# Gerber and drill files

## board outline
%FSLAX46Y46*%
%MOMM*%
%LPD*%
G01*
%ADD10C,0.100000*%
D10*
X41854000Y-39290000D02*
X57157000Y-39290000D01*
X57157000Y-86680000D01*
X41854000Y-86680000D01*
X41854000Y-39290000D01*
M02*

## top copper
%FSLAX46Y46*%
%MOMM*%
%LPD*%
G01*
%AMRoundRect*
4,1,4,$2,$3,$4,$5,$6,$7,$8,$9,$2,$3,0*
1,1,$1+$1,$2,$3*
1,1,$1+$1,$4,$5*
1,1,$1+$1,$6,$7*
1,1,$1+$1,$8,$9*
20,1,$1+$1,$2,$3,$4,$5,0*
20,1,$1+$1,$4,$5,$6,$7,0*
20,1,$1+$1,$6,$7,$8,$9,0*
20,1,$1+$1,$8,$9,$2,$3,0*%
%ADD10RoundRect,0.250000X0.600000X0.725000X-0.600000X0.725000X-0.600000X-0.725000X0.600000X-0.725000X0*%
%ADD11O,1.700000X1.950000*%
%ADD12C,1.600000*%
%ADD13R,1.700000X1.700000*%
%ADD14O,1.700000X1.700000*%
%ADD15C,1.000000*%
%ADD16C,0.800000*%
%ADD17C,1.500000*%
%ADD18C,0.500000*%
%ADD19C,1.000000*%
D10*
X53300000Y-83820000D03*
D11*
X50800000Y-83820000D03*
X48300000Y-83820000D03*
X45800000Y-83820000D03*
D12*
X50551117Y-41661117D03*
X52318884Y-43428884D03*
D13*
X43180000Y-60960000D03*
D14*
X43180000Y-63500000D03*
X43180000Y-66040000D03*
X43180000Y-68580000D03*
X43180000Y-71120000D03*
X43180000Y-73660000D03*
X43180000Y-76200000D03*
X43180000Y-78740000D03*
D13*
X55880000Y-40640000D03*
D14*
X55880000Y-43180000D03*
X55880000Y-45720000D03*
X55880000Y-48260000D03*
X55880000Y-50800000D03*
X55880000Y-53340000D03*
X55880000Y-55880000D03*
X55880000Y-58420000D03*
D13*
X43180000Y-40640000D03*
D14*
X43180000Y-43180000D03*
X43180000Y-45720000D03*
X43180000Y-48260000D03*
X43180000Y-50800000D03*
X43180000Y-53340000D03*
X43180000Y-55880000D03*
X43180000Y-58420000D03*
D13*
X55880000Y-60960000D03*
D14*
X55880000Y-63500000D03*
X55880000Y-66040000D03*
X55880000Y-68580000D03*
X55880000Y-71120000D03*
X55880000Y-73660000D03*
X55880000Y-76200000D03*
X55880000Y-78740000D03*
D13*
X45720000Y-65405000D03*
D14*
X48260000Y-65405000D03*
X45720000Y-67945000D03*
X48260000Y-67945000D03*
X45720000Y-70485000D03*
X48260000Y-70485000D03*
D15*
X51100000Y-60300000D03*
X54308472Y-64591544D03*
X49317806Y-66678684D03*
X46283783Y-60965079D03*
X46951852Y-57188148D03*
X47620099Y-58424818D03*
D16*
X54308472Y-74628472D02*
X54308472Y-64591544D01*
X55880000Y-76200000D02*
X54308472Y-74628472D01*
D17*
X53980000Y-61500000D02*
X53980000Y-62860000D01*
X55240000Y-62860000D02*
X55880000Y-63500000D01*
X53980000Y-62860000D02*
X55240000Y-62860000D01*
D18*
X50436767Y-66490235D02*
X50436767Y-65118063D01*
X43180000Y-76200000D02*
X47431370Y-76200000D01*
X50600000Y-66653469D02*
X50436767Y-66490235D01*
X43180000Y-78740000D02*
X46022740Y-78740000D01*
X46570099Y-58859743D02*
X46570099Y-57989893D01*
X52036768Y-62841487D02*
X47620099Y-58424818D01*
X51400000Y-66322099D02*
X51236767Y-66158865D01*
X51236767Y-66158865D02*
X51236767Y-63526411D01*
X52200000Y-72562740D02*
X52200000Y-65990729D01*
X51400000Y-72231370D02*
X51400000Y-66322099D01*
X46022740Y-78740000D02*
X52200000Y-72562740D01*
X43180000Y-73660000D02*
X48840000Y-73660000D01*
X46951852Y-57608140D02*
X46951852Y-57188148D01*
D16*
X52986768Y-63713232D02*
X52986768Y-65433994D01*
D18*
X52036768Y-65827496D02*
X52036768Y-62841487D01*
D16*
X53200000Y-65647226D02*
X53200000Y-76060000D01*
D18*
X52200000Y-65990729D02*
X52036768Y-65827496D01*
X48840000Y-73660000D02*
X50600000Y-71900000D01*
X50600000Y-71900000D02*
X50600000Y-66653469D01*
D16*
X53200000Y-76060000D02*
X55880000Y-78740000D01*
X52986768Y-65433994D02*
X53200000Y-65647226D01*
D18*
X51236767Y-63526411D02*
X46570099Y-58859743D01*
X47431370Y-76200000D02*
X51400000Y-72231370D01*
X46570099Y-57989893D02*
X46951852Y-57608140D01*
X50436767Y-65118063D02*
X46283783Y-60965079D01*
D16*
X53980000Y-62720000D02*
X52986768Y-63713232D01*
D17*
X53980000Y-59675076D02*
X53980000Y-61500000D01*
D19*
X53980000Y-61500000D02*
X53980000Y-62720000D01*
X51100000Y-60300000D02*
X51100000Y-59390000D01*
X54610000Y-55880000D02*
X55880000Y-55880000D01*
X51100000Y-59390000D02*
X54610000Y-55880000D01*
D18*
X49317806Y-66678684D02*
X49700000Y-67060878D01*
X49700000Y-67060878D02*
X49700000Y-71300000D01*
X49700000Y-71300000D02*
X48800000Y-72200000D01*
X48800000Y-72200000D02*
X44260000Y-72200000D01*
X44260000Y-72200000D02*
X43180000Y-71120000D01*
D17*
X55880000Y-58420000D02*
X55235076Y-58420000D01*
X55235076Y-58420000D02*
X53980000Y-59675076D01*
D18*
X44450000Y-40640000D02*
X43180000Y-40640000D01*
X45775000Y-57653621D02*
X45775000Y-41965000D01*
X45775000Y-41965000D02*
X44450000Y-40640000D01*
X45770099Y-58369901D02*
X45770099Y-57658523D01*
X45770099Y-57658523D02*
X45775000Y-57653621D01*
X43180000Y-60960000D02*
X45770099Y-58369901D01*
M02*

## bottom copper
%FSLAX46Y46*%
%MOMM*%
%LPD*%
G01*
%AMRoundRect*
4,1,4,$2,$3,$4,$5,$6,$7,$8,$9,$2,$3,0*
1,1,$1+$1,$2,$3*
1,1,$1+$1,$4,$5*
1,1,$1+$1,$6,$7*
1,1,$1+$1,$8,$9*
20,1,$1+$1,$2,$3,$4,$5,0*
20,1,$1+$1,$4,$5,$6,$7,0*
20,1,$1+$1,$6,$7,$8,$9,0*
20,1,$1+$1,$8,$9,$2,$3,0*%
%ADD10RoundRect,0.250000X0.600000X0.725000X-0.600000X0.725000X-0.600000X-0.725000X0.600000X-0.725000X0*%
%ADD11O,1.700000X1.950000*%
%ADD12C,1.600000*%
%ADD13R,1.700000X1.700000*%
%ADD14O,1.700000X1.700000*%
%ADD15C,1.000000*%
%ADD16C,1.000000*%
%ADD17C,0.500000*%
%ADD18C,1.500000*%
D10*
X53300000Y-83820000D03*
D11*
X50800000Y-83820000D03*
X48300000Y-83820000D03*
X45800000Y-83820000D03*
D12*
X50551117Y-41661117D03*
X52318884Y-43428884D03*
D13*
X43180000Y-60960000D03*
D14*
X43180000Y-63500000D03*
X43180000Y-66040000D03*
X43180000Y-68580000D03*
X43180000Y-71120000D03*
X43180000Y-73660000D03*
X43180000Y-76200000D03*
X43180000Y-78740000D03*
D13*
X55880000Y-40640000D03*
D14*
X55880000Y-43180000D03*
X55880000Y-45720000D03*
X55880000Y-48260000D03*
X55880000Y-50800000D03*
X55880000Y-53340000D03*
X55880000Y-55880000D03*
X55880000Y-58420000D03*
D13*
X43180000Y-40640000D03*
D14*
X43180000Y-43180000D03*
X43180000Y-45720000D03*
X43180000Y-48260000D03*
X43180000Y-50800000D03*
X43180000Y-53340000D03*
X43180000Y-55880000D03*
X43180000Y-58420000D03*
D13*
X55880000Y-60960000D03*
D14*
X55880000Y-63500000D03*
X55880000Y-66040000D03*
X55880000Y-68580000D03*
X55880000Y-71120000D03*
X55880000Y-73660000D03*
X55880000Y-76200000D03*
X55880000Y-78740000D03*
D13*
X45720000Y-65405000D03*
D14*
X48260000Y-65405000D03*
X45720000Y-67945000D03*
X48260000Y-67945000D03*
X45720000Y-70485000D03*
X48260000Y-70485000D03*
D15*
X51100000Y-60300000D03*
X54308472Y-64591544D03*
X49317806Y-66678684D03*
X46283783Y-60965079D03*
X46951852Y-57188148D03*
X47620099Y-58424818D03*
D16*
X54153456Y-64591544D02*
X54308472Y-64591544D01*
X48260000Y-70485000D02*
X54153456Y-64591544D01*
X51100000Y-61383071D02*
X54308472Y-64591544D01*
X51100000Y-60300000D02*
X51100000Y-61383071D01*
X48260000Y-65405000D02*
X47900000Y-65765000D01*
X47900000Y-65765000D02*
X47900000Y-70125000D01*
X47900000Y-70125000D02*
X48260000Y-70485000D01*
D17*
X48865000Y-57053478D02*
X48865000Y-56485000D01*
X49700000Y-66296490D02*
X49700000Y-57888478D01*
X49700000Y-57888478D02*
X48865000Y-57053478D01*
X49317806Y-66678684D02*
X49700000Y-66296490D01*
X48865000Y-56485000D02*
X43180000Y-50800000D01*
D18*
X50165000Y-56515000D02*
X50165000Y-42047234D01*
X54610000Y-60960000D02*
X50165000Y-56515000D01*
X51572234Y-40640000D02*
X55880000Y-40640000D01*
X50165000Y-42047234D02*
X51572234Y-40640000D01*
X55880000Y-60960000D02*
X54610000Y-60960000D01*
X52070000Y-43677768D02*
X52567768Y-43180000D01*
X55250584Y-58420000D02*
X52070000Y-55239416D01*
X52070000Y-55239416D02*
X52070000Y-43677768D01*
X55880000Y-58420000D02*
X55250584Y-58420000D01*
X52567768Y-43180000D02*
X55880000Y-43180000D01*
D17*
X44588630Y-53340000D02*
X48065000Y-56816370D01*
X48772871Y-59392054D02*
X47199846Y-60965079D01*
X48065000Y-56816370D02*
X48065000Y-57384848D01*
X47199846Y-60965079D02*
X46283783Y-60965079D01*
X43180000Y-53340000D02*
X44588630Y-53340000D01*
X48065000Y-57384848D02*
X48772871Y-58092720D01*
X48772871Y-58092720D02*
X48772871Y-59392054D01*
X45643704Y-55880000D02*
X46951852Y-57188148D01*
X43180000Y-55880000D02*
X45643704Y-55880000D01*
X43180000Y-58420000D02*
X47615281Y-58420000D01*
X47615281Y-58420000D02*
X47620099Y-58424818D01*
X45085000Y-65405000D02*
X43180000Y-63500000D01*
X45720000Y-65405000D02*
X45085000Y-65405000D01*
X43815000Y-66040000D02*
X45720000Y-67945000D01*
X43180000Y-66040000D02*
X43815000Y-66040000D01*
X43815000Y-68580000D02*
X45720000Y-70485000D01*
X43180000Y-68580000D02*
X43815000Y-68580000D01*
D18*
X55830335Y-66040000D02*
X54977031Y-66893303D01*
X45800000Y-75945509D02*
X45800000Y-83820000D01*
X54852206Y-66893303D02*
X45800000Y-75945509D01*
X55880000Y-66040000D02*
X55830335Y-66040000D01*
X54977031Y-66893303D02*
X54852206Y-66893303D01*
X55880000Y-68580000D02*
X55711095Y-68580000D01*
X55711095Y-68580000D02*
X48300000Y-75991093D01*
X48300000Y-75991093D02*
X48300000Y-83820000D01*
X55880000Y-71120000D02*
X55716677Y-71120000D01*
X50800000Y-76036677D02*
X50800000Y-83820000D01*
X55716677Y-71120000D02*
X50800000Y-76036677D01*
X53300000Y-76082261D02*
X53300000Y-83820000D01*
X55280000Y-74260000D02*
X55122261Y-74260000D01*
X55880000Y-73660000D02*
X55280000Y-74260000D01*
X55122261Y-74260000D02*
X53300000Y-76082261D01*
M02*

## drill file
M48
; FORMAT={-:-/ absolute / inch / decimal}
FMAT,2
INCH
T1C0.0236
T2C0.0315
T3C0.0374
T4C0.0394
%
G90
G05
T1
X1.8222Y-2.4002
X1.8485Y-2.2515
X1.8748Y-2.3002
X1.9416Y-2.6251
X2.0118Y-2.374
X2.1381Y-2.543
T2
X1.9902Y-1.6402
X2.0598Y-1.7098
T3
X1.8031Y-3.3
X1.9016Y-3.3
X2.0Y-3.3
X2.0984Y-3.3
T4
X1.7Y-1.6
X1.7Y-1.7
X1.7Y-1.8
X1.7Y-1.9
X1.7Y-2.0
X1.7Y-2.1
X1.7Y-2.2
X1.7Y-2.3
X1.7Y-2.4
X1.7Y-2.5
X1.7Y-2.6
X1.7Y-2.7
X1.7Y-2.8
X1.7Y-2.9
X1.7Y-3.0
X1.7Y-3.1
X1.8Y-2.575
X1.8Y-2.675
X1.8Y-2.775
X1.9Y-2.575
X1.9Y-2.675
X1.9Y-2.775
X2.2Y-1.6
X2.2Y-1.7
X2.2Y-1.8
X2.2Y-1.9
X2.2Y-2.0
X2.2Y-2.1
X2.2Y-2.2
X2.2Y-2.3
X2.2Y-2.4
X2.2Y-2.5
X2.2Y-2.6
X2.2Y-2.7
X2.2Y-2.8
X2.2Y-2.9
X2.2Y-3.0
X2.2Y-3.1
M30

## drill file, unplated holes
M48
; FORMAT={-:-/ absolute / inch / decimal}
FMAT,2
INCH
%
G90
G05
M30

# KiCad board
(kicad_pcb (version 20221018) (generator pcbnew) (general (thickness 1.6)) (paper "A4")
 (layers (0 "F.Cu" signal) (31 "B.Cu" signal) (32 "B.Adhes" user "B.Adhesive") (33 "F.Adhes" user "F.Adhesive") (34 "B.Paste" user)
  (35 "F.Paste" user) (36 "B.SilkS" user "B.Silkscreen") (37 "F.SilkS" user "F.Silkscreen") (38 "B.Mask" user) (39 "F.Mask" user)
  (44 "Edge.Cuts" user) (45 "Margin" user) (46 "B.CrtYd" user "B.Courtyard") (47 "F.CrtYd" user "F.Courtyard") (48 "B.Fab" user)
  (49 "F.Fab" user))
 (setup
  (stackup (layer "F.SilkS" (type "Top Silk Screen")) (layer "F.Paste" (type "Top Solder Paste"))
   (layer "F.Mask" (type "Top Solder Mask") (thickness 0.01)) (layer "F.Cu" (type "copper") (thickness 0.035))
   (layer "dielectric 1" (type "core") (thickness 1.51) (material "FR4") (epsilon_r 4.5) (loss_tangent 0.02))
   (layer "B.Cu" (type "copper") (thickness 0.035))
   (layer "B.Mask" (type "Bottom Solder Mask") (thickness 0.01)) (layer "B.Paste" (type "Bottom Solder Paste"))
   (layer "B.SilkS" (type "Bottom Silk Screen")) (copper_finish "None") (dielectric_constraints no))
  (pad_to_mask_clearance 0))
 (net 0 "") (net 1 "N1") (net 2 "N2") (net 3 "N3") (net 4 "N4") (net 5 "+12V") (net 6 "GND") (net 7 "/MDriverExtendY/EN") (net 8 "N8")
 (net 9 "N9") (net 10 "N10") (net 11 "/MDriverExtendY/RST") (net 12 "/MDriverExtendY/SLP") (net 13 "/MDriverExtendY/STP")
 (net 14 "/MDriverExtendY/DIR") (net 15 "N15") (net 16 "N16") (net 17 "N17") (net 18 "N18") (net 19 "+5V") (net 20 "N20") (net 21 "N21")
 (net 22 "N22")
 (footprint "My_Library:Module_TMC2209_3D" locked (layer "F.Cu") (at 43.18 40.64)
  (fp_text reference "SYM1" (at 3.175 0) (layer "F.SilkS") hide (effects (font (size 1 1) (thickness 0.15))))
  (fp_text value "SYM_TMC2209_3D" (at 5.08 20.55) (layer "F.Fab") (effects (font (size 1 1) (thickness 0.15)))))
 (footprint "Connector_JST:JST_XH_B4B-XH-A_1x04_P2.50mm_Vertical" (layer "F.Cu") (at 53.3 83.82 180)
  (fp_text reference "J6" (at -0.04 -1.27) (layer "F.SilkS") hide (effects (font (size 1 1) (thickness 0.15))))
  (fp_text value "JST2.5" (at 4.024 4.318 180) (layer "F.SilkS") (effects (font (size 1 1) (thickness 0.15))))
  (pad "1" thru_hole roundrect (at 0 0 180) (size 1.7 1.95) (drill 0.95) (layers "*.Cu" "*.Mask") (roundrect_rratio 0.1470588235)
   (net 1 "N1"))
  (pad "2" thru_hole oval (at 2.5 0 180) (size 1.7 1.95) (drill 0.95) (layers "*.Cu" "*.Mask") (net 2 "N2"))
  (pad "3" thru_hole oval (at 5 0 180) (size 1.7 1.95) (drill 0.95) (layers "*.Cu" "*.Mask") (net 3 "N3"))
  (pad "4" thru_hole oval (at 7.5 0 180) (size 1.7 1.95) (drill 0.95) (layers "*.Cu" "*.Mask") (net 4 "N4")))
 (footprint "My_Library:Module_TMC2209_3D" (layer "F.Cu") (at 43.18 60.96)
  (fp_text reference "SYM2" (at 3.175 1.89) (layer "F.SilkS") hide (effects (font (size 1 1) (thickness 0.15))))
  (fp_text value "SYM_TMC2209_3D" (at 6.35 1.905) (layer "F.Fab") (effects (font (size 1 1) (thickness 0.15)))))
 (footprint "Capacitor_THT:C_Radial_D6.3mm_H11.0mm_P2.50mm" (layer "F.Cu") (at 50.551117 41.661117 -45)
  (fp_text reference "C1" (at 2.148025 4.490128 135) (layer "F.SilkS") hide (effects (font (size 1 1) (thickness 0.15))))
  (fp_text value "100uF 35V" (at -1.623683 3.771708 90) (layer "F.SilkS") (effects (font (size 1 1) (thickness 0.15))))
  (pad "1" thru_hole circle (at 0 0 315) (size 1.6 1.6) (drill 0.8) (layers "*.Cu" "*.Mask") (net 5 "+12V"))
  (pad "2" thru_hole circle (at 2.5 0 315) (size 1.6 1.6) (drill 0.8) (layers "*.Cu" "*.Mask") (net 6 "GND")))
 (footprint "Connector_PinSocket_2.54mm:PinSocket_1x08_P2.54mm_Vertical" (layer "F.Cu") (at 43.18 60.96)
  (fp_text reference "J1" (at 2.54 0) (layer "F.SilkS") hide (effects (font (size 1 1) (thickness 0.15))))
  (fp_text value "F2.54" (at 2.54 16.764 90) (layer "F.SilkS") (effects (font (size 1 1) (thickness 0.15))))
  (pad "1" thru_hole rect (at 0 0) (size 1.7 1.7) (drill 1) (layers "*.Cu" "*.Mask") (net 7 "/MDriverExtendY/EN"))
  (pad "2" thru_hole oval (at 0 2.54) (size 1.7 1.7) (drill 1) (layers "*.Cu" "*.Mask") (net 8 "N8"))
  (pad "3" thru_hole oval (at 0 5.08) (size 1.7 1.7) (drill 1) (layers "*.Cu" "*.Mask") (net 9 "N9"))
  (pad "4" thru_hole oval (at 0 7.62) (size 1.7 1.7) (drill 1) (layers "*.Cu" "*.Mask") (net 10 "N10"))
  (pad "5" thru_hole oval (at 0 10.16) (size 1.7 1.7) (drill 1) (layers "*.Cu" "*.Mask") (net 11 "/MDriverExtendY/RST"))
  (pad "6" thru_hole oval (at 0 12.7) (size 1.7 1.7) (drill 1) (layers "*.Cu" "*.Mask") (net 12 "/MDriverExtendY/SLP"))
  (pad "7" thru_hole oval (at 0 15.24) (size 1.7 1.7) (drill 1) (layers "*.Cu" "*.Mask") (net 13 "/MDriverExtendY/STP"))
  (pad "8" thru_hole oval (at 0 17.78) (size 1.7 1.7) (drill 1) (layers "*.Cu" "*.Mask") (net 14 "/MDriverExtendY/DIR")))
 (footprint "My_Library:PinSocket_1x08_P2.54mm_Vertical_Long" (layer "F.Cu") (at 55.88 40.64)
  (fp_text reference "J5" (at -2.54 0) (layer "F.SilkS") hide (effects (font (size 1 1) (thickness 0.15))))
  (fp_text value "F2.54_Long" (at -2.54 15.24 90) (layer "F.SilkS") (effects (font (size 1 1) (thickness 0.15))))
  (pad "1" thru_hole rect (at 0 0) (size 1.7 1.7) (drill 1) (layers "*.Cu" "*.Mask") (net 5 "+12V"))
  (pad "2" thru_hole oval (at 0 2.54) (size 1.7 1.7) (drill 1) (layers "*.Cu" "*.Mask") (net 6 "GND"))
  (pad "3" thru_hole oval (at 0 5.08) (size 1.7 1.7) (drill 1) (layers "*.Cu" "*.Mask") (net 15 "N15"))
  (pad "4" thru_hole oval (at 0 7.62) (size 1.7 1.7) (drill 1) (layers "*.Cu" "*.Mask") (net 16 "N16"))
  (pad "5" thru_hole oval (at 0 10.16) (size 1.7 1.7) (drill 1) (layers "*.Cu" "*.Mask") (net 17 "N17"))
  (pad "6" thru_hole oval (at 0 12.7) (size 1.7 1.7) (drill 1) (layers "*.Cu" "*.Mask") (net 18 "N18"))
  (pad "7" thru_hole oval (at 0 15.24) (size 1.7 1.7) (drill 1) (layers "*.Cu" "*.Mask") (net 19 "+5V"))
  (pad "8" thru_hole oval (at 0 17.78) (size 1.7 1.7) (drill 1) (layers "*.Cu" "*.Mask") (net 6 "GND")))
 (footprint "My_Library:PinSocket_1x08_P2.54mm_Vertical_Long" (layer "F.Cu") (at 43.18 40.64)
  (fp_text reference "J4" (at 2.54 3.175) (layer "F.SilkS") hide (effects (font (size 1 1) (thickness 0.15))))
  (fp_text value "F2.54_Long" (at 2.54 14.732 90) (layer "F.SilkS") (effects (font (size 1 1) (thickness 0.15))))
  (pad "1" thru_hole rect (at 0 0) (size 1.7 1.7) (drill 1) (layers "*.Cu" "*.Mask") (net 7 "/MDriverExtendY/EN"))
  (pad "2" thru_hole oval (at 0 2.54) (size 1.7 1.7) (drill 1) (layers "*.Cu" "*.Mask") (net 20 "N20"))
  (pad "3" thru_hole oval (at 0 5.08) (size 1.7 1.7) (drill 1) (layers "*.Cu" "*.Mask") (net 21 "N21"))
  (pad "4" thru_hole oval (at 0 7.62) (size 1.7 1.7) (drill 1) (layers "*.Cu" "*.Mask") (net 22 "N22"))
  (pad "5" thru_hole oval (at 0 10.16) (size 1.7 1.7) (drill 1) (layers "*.Cu" "*.Mask") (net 11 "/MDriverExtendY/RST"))
  (pad "6" thru_hole oval (at 0 12.7) (size 1.7 1.7) (drill 1) (layers "*.Cu" "*.Mask") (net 12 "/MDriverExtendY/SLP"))
  (pad "7" thru_hole oval (at 0 15.24) (size 1.7 1.7) (drill 1) (layers "*.Cu" "*.Mask") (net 13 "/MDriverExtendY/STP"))
  (pad "8" thru_hole oval (at 0 17.78) (size 1.7 1.7) (drill 1) (layers "*.Cu" "*.Mask") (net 14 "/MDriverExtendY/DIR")))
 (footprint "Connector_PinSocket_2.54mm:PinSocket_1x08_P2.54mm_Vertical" (layer "F.Cu") (at 55.88 60.96)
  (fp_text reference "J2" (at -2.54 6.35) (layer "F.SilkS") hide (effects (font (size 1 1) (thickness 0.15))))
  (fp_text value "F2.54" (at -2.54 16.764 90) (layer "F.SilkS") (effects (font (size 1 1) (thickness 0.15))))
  (pad "1" thru_hole rect (at 0 0) (size 1.7 1.7) (drill 1) (layers "*.Cu" "*.Mask") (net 5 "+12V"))
  (pad "2" thru_hole oval (at 0 2.54) (size 1.7 1.7) (drill 1) (layers "*.Cu" "*.Mask") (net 6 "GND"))
  (pad "3" thru_hole oval (at 0 5.08) (size 1.7 1.7) (drill 1) (layers "*.Cu" "*.Mask") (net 4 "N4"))
  (pad "4" thru_hole oval (at 0 7.62) (size 1.7 1.7) (drill 1) (layers "*.Cu" "*.Mask") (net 3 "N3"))
  (pad "5" thru_hole oval (at 0 10.16) (size 1.7 1.7) (drill 1) (layers "*.Cu" "*.Mask") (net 2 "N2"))
  (pad "6" thru_hole oval (at 0 12.7) (size 1.7 1.7) (drill 1) (layers "*.Cu" "*.Mask") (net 1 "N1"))
  (pad "7" thru_hole oval (at 0 15.24) (size 1.7 1.7) (drill 1) (layers "*.Cu" "*.Mask") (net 19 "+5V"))
  (pad "8" thru_hole oval (at 0 17.78) (size 1.7 1.7) (drill 1) (layers "*.Cu" "*.Mask") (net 6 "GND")))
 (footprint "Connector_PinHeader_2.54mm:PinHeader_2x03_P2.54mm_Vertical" (layer "F.Cu") (at 45.72 65.405)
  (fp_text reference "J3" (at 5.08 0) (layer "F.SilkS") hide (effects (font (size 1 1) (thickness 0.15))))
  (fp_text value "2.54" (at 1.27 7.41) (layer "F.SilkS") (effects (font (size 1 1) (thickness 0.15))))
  (pad "1" thru_hole rect (at 0 0) (size 1.7 1.7) (drill 1) (layers "*.Cu" "*.Mask") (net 8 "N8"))
  (pad "2" thru_hole oval (at 2.54 0) (size 1.7 1.7) (drill 1) (layers "*.Cu" "*.Mask") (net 19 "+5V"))
  (pad "3" thru_hole oval (at 0 2.54) (size 1.7 1.7) (drill 1) (layers "*.Cu" "*.Mask") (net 9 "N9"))
  (pad "4" thru_hole oval (at 2.54 2.54) (size 1.7 1.7) (drill 1) (layers "*.Cu" "*.Mask") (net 19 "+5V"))
  (pad "5" thru_hole oval (at 0 5.08) (size 1.7 1.7) (drill 1) (layers "*.Cu" "*.Mask") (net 10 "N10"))
  (pad "6" thru_hole oval (at 2.54 5.08) (size 1.7 1.7) (drill 1) (layers "*.Cu" "*.Mask") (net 19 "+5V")))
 (gr_rect (start 41.854 39.29) (end 57.157 86.68) (stroke (width 0.1) (type default)) (fill none) (layer "Edge.Cuts"))
 (segment (start 50.165 56.515) (end 50.165 42.047234) (width 1.5) (layer "B.Cu") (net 5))
 (segment (start 54.61 60.96) (end 50.165 56.515) (width 1.5) (layer "B.Cu") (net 5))
 (segment (start 51.572234 40.64) (end 55.88 40.64) (width 1.5) (layer "B.Cu") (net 5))
 (segment (start 50.165 42.047234) (end 51.572234 40.64) (width 1.5) (layer "B.Cu") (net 5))
 (segment (start 55.88 60.96) (end 54.61 60.96) (width 1.5) (layer "B.Cu") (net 5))
 (segment (start 53.2 65.647226) (end 53.2 76.06) (width 0.8) (layer "F.Cu") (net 6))
 (segment (start 55.88 58.42) (end 55.235076 58.42) (width 1.5) (layer "F.Cu") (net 6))
 (segment (start 53.98 59.675076) (end 53.98 61.5) (width 1.5) (layer "F.Cu") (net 6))
 (segment (start 53.98 62.86) (end 55.24 62.86) (width 1.5) (layer "F.Cu") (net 6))
 (segment (start 53.98 62.72) (end 52.986768 63.713232) (width 0.8) (layer "F.Cu") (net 6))
 (segment (start 52.986768 65.433994) (end 53.2 65.647226) (width 0.8) (layer "F.Cu") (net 6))
 (segment (start 53.2 76.06) (end 55.88 78.74) (width 0.8) (layer "F.Cu") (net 6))
 (segment (start 53.98 61.5) (end 53.98 62.86) (width 1.5) (layer "F.Cu") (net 6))
 (segment (start 55.235076 58.42) (end 53.98 59.675076) (width 1.5) (layer "F.Cu") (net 6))
 (segment (start 52.986768 63.713232) (end 52.986768 65.433994) (width 0.8) (layer "F.Cu") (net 6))
 (segment (start 55.24 62.86) (end 55.88 63.5) (width 1.5) (layer "F.Cu") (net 6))
 (segment (start 53.98 61.5) (end 53.98 62.72) (width 1) (layer "F.Cu") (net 6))
 (segment (start 52.07 43.677768) (end 52.567768 43.18) (width 1.5) (layer "B.Cu") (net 6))
 (segment (start 55.250584 58.42) (end 52.07 55.239416) (width 1.5) (layer "B.Cu") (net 6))
 (segment (start 52.07 55.239416) (end 52.07 43.677768) (width 1.5) (layer "B.Cu") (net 6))
 (segment (start 55.88 58.42) (end 55.250584 58.42) (width 1.5) (layer "B.Cu") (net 6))
 (segment (start 52.567768 43.18) (end 55.88 43.18) (width 1.5) (layer "B.Cu") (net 6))
 (segment (start 54.61 55.88) (end 55.88 55.88) (width 1) (layer "F.Cu") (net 19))
 (segment (start 51.1 59.39) (end 54.61 55.88) (width 1) (layer "F.Cu") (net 19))
 (segment (start 51.1 60.3) (end 51.1 59.39) (width 1) (layer "F.Cu") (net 19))
 (segment (start 54.308472 74.628472) (end 54.308472 64.591544) (width 0.8) (layer "F.Cu") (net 19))
 (segment (start 55.88 76.2) (end 54.308472 74.628472) (width 0.8) (layer "F.Cu") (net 19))
 (via (at 54.308472 64.591544) (size 1) (drill 0.6) (layers "F.Cu" "B.Cu") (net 19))
 (via (at 51.1 60.3) (size 1) (drill 0.6) (layers "F.Cu" "B.Cu") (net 19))
 (segment (start 48.26 65.405) (end 47.9 65.765) (width 1) (layer "B.Cu") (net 19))
 (segment (start 51.1 60.3) (end 51.1 61.383071) (width 1) (layer "B.Cu") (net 19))
 (segment (start 51.1 61.383071) (end 54.308472 64.591544) (width 1) (layer "B.Cu") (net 19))
 (segment (start 48.26 70.485) (end 54.153456 64.591544) (width 1) (layer "B.Cu") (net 19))
 (segment (start 47.9 70.125) (end 48.26 70.485) (width 1) (layer "B.Cu") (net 19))
 (segment (start 54.153456 64.591544) (end 54.308472 64.591544) (width 1) (layer "B.Cu") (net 19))
 (segment (start 47.9 65.765) (end 47.9 70.125) (width 1) (layer "B.Cu") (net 19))
 (segment (start 44.45 40.64) (end 43.18 40.64) (width 0.5) (layer "F.Cu") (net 7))
 (segment (start 45.775 57.653621) (end 45.775 41.965) (width 0.5) (layer "F.Cu") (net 7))
 (segment (start 45.775 41.965) (end 44.45 40.64) (width 0.5) (layer "F.Cu") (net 7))
 (segment (start 45.770099 58.369901) (end 45.770099 57.658523) (width 0.5) (layer "F.Cu") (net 7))
 (segment (start 45.770099 57.658523) (end 45.775 57.653621) (width 0.5) (layer "F.Cu") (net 7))
 (segment (start 43.18 60.96) (end 45.770099 58.369901) (width 0.5) (layer "F.Cu") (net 7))
 (segment (start 44.26 72.2) (end 43.18 71.12) (width 0.5) (layer "F.Cu") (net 11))
 (segment (start 49.7 71.3) (end 48.8 72.2) (width 0.5) (layer "F.Cu") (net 11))
 (segment (start 49.317806 66.678684) (end 49.7 67.060878) (width 0.5) (layer "F.Cu") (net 11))
 (segment (start 48.8 72.2) (end 44.26 72.2) (width 0.5) (layer "F.Cu") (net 11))
 (segment (start 49.7 67.060878) (end 49.7 71.3) (width 0.5) (layer "F.Cu") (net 11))
 (via (at 49.317806 66.678684) (size 1) (drill 0.6) (layers "F.Cu" "B.Cu") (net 11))
 (segment (start 49.7 57.888478) (end 48.865 57.053478) (width 0.5) (layer "B.Cu") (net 11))
 (segment (start 49.7 66.29649) (end 49.7 57.888478) (width 0.5) (layer "B.Cu") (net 11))
 (segment (start 48.865 57.053478) (end 48.865 56.485) (width 0.5) (layer "B.Cu") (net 11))
 (segment (start 49.317806 66.678684) (end 49.7 66.29649) (width 0.5) (layer "B.Cu") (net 11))
 (segment (start 48.865 56.485) (end 43.18 50.8) (width 0.5) (layer "B.Cu") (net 11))
 (segment (start 50.436767 65.118063) (end 46.283783 60.965079) (width 0.5) (layer "F.Cu") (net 12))
 (segment (start 50.6 66.653469) (end 50.436767 66.490235) (width 0.5) (layer "F.Cu") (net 12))
 (segment (start 43.18 73.66) (end 48.84 73.66) (width 0.5) (layer "F.Cu") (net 12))
 (segment (start 50.436767 66.490235) (end 50.436767 65.118063) (width 0.5) (layer "F.Cu") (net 12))
 (segment (start 50.6 71.9) (end 50.6 66.653469) (width 0.5) (layer "F.Cu") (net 12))
 (segment (start 48.84 73.66) (end 50.6 71.9) (width 0.5) (layer "F.Cu") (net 12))
 (via (at 46.283783 60.965079) (size 1) (drill 0.6) (layers "F.Cu" "B.Cu") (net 12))
 (segment (start 44.58863 53.34) (end 48.065 56.81637) (width 0.5) (layer "B.Cu") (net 12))
 (segment (start 48.772871 59.392054) (end 47.199846 60.965079) (width 0.5) (layer "B.Cu") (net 12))
 (segment (start 48.065 56.81637) (end 48.065 57.384848) (width 0.5) (layer "B.Cu") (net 12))
 (segment (start 47.199846 60.965079) (end 46.283783 60.965079) (width 0.5) (layer "B.Cu") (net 12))
 (segment (start 43.18 53.34) (end 44.58863 53.34) (width 0.5) (layer "B.Cu") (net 12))
 (segment (start 48.065 57.384848) (end 48.772871 58.09272) (width 0.5) (layer "B.Cu") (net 12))
 (segment (start 48.772871 58.09272) (end 48.772871 59.392054) (width 0.5) (layer "B.Cu") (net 12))
 (segment (start 51.236767 63.526411) (end 46.570099 58.859743) (width 0.5) (layer "F.Cu") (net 13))
 (segment (start 51.236767 66.158865) (end 51.236767 63.526411) (width 0.5) (layer "F.Cu") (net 13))
 (segment (start 46.570099 57.989893) (end 46.951852 57.60814) (width 0.5) (layer "F.Cu") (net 13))
 (segment (start 51.4 66.322099) (end 51.236767 66.158865) (width 0.5) (layer "F.Cu") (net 13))
 (segment (start 46.951852 57.60814) (end 46.951852 57.188148) (width 0.5) (layer "F.Cu") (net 13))
 (segment (start 51.4 72.23137) (end 51.4 66.322099) (width 0.5) (layer "F.Cu") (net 13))
 (segment (start 43.18 76.2) (end 47.43137 76.2) (width 0.5) (layer "F.Cu") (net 13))
 (segment (start 47.43137 76.2) (end 51.4 72.23137) (width 0.5) (layer "F.Cu") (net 13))
 (segment (start 46.570099 58.859743) (end 46.570099 57.989893) (width 0.5) (layer "F.Cu") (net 13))
 (via (at 46.951852 57.188148) (size 1) (drill 0.6) (layers "F.Cu" "B.Cu") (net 13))
 (segment (start 45.643704 55.88) (end 46.951852 57.188148) (width 0.5) (layer "B.Cu") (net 13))
 (segment (start 43.18 55.88) (end 45.643704 55.88) (width 0.5) (layer "B.Cu") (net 13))
 (segment (start 43.18 78.74) (end 46.02274 78.74) (width 0.5) (layer "F.Cu") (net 14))
 (segment (start 52.2 72.56274) (end 52.2 65.990729) (width 0.5) (layer "F.Cu") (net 14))
 (segment (start 52.036768 62.841487) (end 47.620099 58.424818) (width 0.5) (layer "F.Cu") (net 14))
 (segment (start 46.02274 78.74) (end 52.2 72.56274) (width 0.5) (layer "F.Cu") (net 14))
 (segment (start 52.2 65.990729) (end 52.036768 65.827496) (width 0.5) (layer "F.Cu") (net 14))
 (segment (start 52.036768 65.827496) (end 52.036768 62.841487) (width 0.5) (layer "F.Cu") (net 14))
 (via (at 47.620099 58.424818) (size 1) (drill 0.6) (layers "F.Cu" "B.Cu") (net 14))
 (segment (start 43.18 58.42) (end 47.615281 58.42) (width 0.5) (layer "B.Cu") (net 14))
 (segment (start 47.615281 58.42) (end 47.620099 58.424818) (width 0.5) (layer "B.Cu") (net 14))
 (segment (start 45.085 65.405) (end 43.18 63.5) (width 0.5) (layer "B.Cu") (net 8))
 (segment (start 45.72 65.405) (end 45.085 65.405) (width 0.5) (layer "B.Cu") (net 8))
 (segment (start 43.815 66.04) (end 45.72 67.945) (width 0.5) (layer "B.Cu") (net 9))
 (segment (start 43.18 66.04) (end 43.815 66.04) (width 0.5) (layer "B.Cu") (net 9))
 (segment (start 43.815 68.58) (end 45.72 70.485) (width 0.5) (layer "B.Cu") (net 10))
 (segment (start 43.18 68.58) (end 43.815 68.58) (width 0.5) (layer "B.Cu") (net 10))
 (segment (start 55.830335 66.04) (end 54.977031 66.893303) (width 1.5) (layer "B.Cu") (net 4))
 (segment (start 45.8 75.945509) (end 45.8 83.82) (width 1.5) (layer "B.Cu") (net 4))
 (segment (start 54.852206 66.893303) (end 45.8 75.945509) (width 1.5) (layer "B.Cu") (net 4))
 (segment (start 55.88 66.04) (end 55.830335 66.04) (width 1.5) (layer "B.Cu") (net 4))
 (segment (start 54.977031 66.893303) (end 54.852206 66.893303) (width 1.5) (layer "B.Cu") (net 4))
 (segment (start 55.88 68.58) (end 55.711095 68.58) (width 1.5) (layer "B.Cu") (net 3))
 (segment (start 55.711095 68.58) (end 48.3 75.991093) (width 1.5) (layer "B.Cu") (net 3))
 (segment (start 48.3 75.991093) (end 48.3 83.82) (width 1.5) (layer "B.Cu") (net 3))
 (segment (start 55.88 71.12) (end 55.716677 71.12) (width 1.5) (layer "B.Cu") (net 2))
 (segment (start 50.8 76.036677) (end 50.8 83.82) (width 1.5) (layer "B.Cu") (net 2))
 (segment (start 55.716677 71.12) (end 50.8 76.036677) (width 1.5) (layer "B.Cu") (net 2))
 (segment (start 53.3 76.082261) (end 53.3 83.82) (width 1.5) (layer "B.Cu") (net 1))
 (segment (start 55.28 74.26) (end 55.122261 74.26) (width 1.5) (layer "B.Cu") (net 1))
 (segment (start 55.88 73.66) (end 55.28 74.26) (width 1.5) (layer "B.Cu") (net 1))
 (segment (start 55.122261 74.26) (end 53.3 76.082261) (width 1.5) (layer "B.Cu") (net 1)))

